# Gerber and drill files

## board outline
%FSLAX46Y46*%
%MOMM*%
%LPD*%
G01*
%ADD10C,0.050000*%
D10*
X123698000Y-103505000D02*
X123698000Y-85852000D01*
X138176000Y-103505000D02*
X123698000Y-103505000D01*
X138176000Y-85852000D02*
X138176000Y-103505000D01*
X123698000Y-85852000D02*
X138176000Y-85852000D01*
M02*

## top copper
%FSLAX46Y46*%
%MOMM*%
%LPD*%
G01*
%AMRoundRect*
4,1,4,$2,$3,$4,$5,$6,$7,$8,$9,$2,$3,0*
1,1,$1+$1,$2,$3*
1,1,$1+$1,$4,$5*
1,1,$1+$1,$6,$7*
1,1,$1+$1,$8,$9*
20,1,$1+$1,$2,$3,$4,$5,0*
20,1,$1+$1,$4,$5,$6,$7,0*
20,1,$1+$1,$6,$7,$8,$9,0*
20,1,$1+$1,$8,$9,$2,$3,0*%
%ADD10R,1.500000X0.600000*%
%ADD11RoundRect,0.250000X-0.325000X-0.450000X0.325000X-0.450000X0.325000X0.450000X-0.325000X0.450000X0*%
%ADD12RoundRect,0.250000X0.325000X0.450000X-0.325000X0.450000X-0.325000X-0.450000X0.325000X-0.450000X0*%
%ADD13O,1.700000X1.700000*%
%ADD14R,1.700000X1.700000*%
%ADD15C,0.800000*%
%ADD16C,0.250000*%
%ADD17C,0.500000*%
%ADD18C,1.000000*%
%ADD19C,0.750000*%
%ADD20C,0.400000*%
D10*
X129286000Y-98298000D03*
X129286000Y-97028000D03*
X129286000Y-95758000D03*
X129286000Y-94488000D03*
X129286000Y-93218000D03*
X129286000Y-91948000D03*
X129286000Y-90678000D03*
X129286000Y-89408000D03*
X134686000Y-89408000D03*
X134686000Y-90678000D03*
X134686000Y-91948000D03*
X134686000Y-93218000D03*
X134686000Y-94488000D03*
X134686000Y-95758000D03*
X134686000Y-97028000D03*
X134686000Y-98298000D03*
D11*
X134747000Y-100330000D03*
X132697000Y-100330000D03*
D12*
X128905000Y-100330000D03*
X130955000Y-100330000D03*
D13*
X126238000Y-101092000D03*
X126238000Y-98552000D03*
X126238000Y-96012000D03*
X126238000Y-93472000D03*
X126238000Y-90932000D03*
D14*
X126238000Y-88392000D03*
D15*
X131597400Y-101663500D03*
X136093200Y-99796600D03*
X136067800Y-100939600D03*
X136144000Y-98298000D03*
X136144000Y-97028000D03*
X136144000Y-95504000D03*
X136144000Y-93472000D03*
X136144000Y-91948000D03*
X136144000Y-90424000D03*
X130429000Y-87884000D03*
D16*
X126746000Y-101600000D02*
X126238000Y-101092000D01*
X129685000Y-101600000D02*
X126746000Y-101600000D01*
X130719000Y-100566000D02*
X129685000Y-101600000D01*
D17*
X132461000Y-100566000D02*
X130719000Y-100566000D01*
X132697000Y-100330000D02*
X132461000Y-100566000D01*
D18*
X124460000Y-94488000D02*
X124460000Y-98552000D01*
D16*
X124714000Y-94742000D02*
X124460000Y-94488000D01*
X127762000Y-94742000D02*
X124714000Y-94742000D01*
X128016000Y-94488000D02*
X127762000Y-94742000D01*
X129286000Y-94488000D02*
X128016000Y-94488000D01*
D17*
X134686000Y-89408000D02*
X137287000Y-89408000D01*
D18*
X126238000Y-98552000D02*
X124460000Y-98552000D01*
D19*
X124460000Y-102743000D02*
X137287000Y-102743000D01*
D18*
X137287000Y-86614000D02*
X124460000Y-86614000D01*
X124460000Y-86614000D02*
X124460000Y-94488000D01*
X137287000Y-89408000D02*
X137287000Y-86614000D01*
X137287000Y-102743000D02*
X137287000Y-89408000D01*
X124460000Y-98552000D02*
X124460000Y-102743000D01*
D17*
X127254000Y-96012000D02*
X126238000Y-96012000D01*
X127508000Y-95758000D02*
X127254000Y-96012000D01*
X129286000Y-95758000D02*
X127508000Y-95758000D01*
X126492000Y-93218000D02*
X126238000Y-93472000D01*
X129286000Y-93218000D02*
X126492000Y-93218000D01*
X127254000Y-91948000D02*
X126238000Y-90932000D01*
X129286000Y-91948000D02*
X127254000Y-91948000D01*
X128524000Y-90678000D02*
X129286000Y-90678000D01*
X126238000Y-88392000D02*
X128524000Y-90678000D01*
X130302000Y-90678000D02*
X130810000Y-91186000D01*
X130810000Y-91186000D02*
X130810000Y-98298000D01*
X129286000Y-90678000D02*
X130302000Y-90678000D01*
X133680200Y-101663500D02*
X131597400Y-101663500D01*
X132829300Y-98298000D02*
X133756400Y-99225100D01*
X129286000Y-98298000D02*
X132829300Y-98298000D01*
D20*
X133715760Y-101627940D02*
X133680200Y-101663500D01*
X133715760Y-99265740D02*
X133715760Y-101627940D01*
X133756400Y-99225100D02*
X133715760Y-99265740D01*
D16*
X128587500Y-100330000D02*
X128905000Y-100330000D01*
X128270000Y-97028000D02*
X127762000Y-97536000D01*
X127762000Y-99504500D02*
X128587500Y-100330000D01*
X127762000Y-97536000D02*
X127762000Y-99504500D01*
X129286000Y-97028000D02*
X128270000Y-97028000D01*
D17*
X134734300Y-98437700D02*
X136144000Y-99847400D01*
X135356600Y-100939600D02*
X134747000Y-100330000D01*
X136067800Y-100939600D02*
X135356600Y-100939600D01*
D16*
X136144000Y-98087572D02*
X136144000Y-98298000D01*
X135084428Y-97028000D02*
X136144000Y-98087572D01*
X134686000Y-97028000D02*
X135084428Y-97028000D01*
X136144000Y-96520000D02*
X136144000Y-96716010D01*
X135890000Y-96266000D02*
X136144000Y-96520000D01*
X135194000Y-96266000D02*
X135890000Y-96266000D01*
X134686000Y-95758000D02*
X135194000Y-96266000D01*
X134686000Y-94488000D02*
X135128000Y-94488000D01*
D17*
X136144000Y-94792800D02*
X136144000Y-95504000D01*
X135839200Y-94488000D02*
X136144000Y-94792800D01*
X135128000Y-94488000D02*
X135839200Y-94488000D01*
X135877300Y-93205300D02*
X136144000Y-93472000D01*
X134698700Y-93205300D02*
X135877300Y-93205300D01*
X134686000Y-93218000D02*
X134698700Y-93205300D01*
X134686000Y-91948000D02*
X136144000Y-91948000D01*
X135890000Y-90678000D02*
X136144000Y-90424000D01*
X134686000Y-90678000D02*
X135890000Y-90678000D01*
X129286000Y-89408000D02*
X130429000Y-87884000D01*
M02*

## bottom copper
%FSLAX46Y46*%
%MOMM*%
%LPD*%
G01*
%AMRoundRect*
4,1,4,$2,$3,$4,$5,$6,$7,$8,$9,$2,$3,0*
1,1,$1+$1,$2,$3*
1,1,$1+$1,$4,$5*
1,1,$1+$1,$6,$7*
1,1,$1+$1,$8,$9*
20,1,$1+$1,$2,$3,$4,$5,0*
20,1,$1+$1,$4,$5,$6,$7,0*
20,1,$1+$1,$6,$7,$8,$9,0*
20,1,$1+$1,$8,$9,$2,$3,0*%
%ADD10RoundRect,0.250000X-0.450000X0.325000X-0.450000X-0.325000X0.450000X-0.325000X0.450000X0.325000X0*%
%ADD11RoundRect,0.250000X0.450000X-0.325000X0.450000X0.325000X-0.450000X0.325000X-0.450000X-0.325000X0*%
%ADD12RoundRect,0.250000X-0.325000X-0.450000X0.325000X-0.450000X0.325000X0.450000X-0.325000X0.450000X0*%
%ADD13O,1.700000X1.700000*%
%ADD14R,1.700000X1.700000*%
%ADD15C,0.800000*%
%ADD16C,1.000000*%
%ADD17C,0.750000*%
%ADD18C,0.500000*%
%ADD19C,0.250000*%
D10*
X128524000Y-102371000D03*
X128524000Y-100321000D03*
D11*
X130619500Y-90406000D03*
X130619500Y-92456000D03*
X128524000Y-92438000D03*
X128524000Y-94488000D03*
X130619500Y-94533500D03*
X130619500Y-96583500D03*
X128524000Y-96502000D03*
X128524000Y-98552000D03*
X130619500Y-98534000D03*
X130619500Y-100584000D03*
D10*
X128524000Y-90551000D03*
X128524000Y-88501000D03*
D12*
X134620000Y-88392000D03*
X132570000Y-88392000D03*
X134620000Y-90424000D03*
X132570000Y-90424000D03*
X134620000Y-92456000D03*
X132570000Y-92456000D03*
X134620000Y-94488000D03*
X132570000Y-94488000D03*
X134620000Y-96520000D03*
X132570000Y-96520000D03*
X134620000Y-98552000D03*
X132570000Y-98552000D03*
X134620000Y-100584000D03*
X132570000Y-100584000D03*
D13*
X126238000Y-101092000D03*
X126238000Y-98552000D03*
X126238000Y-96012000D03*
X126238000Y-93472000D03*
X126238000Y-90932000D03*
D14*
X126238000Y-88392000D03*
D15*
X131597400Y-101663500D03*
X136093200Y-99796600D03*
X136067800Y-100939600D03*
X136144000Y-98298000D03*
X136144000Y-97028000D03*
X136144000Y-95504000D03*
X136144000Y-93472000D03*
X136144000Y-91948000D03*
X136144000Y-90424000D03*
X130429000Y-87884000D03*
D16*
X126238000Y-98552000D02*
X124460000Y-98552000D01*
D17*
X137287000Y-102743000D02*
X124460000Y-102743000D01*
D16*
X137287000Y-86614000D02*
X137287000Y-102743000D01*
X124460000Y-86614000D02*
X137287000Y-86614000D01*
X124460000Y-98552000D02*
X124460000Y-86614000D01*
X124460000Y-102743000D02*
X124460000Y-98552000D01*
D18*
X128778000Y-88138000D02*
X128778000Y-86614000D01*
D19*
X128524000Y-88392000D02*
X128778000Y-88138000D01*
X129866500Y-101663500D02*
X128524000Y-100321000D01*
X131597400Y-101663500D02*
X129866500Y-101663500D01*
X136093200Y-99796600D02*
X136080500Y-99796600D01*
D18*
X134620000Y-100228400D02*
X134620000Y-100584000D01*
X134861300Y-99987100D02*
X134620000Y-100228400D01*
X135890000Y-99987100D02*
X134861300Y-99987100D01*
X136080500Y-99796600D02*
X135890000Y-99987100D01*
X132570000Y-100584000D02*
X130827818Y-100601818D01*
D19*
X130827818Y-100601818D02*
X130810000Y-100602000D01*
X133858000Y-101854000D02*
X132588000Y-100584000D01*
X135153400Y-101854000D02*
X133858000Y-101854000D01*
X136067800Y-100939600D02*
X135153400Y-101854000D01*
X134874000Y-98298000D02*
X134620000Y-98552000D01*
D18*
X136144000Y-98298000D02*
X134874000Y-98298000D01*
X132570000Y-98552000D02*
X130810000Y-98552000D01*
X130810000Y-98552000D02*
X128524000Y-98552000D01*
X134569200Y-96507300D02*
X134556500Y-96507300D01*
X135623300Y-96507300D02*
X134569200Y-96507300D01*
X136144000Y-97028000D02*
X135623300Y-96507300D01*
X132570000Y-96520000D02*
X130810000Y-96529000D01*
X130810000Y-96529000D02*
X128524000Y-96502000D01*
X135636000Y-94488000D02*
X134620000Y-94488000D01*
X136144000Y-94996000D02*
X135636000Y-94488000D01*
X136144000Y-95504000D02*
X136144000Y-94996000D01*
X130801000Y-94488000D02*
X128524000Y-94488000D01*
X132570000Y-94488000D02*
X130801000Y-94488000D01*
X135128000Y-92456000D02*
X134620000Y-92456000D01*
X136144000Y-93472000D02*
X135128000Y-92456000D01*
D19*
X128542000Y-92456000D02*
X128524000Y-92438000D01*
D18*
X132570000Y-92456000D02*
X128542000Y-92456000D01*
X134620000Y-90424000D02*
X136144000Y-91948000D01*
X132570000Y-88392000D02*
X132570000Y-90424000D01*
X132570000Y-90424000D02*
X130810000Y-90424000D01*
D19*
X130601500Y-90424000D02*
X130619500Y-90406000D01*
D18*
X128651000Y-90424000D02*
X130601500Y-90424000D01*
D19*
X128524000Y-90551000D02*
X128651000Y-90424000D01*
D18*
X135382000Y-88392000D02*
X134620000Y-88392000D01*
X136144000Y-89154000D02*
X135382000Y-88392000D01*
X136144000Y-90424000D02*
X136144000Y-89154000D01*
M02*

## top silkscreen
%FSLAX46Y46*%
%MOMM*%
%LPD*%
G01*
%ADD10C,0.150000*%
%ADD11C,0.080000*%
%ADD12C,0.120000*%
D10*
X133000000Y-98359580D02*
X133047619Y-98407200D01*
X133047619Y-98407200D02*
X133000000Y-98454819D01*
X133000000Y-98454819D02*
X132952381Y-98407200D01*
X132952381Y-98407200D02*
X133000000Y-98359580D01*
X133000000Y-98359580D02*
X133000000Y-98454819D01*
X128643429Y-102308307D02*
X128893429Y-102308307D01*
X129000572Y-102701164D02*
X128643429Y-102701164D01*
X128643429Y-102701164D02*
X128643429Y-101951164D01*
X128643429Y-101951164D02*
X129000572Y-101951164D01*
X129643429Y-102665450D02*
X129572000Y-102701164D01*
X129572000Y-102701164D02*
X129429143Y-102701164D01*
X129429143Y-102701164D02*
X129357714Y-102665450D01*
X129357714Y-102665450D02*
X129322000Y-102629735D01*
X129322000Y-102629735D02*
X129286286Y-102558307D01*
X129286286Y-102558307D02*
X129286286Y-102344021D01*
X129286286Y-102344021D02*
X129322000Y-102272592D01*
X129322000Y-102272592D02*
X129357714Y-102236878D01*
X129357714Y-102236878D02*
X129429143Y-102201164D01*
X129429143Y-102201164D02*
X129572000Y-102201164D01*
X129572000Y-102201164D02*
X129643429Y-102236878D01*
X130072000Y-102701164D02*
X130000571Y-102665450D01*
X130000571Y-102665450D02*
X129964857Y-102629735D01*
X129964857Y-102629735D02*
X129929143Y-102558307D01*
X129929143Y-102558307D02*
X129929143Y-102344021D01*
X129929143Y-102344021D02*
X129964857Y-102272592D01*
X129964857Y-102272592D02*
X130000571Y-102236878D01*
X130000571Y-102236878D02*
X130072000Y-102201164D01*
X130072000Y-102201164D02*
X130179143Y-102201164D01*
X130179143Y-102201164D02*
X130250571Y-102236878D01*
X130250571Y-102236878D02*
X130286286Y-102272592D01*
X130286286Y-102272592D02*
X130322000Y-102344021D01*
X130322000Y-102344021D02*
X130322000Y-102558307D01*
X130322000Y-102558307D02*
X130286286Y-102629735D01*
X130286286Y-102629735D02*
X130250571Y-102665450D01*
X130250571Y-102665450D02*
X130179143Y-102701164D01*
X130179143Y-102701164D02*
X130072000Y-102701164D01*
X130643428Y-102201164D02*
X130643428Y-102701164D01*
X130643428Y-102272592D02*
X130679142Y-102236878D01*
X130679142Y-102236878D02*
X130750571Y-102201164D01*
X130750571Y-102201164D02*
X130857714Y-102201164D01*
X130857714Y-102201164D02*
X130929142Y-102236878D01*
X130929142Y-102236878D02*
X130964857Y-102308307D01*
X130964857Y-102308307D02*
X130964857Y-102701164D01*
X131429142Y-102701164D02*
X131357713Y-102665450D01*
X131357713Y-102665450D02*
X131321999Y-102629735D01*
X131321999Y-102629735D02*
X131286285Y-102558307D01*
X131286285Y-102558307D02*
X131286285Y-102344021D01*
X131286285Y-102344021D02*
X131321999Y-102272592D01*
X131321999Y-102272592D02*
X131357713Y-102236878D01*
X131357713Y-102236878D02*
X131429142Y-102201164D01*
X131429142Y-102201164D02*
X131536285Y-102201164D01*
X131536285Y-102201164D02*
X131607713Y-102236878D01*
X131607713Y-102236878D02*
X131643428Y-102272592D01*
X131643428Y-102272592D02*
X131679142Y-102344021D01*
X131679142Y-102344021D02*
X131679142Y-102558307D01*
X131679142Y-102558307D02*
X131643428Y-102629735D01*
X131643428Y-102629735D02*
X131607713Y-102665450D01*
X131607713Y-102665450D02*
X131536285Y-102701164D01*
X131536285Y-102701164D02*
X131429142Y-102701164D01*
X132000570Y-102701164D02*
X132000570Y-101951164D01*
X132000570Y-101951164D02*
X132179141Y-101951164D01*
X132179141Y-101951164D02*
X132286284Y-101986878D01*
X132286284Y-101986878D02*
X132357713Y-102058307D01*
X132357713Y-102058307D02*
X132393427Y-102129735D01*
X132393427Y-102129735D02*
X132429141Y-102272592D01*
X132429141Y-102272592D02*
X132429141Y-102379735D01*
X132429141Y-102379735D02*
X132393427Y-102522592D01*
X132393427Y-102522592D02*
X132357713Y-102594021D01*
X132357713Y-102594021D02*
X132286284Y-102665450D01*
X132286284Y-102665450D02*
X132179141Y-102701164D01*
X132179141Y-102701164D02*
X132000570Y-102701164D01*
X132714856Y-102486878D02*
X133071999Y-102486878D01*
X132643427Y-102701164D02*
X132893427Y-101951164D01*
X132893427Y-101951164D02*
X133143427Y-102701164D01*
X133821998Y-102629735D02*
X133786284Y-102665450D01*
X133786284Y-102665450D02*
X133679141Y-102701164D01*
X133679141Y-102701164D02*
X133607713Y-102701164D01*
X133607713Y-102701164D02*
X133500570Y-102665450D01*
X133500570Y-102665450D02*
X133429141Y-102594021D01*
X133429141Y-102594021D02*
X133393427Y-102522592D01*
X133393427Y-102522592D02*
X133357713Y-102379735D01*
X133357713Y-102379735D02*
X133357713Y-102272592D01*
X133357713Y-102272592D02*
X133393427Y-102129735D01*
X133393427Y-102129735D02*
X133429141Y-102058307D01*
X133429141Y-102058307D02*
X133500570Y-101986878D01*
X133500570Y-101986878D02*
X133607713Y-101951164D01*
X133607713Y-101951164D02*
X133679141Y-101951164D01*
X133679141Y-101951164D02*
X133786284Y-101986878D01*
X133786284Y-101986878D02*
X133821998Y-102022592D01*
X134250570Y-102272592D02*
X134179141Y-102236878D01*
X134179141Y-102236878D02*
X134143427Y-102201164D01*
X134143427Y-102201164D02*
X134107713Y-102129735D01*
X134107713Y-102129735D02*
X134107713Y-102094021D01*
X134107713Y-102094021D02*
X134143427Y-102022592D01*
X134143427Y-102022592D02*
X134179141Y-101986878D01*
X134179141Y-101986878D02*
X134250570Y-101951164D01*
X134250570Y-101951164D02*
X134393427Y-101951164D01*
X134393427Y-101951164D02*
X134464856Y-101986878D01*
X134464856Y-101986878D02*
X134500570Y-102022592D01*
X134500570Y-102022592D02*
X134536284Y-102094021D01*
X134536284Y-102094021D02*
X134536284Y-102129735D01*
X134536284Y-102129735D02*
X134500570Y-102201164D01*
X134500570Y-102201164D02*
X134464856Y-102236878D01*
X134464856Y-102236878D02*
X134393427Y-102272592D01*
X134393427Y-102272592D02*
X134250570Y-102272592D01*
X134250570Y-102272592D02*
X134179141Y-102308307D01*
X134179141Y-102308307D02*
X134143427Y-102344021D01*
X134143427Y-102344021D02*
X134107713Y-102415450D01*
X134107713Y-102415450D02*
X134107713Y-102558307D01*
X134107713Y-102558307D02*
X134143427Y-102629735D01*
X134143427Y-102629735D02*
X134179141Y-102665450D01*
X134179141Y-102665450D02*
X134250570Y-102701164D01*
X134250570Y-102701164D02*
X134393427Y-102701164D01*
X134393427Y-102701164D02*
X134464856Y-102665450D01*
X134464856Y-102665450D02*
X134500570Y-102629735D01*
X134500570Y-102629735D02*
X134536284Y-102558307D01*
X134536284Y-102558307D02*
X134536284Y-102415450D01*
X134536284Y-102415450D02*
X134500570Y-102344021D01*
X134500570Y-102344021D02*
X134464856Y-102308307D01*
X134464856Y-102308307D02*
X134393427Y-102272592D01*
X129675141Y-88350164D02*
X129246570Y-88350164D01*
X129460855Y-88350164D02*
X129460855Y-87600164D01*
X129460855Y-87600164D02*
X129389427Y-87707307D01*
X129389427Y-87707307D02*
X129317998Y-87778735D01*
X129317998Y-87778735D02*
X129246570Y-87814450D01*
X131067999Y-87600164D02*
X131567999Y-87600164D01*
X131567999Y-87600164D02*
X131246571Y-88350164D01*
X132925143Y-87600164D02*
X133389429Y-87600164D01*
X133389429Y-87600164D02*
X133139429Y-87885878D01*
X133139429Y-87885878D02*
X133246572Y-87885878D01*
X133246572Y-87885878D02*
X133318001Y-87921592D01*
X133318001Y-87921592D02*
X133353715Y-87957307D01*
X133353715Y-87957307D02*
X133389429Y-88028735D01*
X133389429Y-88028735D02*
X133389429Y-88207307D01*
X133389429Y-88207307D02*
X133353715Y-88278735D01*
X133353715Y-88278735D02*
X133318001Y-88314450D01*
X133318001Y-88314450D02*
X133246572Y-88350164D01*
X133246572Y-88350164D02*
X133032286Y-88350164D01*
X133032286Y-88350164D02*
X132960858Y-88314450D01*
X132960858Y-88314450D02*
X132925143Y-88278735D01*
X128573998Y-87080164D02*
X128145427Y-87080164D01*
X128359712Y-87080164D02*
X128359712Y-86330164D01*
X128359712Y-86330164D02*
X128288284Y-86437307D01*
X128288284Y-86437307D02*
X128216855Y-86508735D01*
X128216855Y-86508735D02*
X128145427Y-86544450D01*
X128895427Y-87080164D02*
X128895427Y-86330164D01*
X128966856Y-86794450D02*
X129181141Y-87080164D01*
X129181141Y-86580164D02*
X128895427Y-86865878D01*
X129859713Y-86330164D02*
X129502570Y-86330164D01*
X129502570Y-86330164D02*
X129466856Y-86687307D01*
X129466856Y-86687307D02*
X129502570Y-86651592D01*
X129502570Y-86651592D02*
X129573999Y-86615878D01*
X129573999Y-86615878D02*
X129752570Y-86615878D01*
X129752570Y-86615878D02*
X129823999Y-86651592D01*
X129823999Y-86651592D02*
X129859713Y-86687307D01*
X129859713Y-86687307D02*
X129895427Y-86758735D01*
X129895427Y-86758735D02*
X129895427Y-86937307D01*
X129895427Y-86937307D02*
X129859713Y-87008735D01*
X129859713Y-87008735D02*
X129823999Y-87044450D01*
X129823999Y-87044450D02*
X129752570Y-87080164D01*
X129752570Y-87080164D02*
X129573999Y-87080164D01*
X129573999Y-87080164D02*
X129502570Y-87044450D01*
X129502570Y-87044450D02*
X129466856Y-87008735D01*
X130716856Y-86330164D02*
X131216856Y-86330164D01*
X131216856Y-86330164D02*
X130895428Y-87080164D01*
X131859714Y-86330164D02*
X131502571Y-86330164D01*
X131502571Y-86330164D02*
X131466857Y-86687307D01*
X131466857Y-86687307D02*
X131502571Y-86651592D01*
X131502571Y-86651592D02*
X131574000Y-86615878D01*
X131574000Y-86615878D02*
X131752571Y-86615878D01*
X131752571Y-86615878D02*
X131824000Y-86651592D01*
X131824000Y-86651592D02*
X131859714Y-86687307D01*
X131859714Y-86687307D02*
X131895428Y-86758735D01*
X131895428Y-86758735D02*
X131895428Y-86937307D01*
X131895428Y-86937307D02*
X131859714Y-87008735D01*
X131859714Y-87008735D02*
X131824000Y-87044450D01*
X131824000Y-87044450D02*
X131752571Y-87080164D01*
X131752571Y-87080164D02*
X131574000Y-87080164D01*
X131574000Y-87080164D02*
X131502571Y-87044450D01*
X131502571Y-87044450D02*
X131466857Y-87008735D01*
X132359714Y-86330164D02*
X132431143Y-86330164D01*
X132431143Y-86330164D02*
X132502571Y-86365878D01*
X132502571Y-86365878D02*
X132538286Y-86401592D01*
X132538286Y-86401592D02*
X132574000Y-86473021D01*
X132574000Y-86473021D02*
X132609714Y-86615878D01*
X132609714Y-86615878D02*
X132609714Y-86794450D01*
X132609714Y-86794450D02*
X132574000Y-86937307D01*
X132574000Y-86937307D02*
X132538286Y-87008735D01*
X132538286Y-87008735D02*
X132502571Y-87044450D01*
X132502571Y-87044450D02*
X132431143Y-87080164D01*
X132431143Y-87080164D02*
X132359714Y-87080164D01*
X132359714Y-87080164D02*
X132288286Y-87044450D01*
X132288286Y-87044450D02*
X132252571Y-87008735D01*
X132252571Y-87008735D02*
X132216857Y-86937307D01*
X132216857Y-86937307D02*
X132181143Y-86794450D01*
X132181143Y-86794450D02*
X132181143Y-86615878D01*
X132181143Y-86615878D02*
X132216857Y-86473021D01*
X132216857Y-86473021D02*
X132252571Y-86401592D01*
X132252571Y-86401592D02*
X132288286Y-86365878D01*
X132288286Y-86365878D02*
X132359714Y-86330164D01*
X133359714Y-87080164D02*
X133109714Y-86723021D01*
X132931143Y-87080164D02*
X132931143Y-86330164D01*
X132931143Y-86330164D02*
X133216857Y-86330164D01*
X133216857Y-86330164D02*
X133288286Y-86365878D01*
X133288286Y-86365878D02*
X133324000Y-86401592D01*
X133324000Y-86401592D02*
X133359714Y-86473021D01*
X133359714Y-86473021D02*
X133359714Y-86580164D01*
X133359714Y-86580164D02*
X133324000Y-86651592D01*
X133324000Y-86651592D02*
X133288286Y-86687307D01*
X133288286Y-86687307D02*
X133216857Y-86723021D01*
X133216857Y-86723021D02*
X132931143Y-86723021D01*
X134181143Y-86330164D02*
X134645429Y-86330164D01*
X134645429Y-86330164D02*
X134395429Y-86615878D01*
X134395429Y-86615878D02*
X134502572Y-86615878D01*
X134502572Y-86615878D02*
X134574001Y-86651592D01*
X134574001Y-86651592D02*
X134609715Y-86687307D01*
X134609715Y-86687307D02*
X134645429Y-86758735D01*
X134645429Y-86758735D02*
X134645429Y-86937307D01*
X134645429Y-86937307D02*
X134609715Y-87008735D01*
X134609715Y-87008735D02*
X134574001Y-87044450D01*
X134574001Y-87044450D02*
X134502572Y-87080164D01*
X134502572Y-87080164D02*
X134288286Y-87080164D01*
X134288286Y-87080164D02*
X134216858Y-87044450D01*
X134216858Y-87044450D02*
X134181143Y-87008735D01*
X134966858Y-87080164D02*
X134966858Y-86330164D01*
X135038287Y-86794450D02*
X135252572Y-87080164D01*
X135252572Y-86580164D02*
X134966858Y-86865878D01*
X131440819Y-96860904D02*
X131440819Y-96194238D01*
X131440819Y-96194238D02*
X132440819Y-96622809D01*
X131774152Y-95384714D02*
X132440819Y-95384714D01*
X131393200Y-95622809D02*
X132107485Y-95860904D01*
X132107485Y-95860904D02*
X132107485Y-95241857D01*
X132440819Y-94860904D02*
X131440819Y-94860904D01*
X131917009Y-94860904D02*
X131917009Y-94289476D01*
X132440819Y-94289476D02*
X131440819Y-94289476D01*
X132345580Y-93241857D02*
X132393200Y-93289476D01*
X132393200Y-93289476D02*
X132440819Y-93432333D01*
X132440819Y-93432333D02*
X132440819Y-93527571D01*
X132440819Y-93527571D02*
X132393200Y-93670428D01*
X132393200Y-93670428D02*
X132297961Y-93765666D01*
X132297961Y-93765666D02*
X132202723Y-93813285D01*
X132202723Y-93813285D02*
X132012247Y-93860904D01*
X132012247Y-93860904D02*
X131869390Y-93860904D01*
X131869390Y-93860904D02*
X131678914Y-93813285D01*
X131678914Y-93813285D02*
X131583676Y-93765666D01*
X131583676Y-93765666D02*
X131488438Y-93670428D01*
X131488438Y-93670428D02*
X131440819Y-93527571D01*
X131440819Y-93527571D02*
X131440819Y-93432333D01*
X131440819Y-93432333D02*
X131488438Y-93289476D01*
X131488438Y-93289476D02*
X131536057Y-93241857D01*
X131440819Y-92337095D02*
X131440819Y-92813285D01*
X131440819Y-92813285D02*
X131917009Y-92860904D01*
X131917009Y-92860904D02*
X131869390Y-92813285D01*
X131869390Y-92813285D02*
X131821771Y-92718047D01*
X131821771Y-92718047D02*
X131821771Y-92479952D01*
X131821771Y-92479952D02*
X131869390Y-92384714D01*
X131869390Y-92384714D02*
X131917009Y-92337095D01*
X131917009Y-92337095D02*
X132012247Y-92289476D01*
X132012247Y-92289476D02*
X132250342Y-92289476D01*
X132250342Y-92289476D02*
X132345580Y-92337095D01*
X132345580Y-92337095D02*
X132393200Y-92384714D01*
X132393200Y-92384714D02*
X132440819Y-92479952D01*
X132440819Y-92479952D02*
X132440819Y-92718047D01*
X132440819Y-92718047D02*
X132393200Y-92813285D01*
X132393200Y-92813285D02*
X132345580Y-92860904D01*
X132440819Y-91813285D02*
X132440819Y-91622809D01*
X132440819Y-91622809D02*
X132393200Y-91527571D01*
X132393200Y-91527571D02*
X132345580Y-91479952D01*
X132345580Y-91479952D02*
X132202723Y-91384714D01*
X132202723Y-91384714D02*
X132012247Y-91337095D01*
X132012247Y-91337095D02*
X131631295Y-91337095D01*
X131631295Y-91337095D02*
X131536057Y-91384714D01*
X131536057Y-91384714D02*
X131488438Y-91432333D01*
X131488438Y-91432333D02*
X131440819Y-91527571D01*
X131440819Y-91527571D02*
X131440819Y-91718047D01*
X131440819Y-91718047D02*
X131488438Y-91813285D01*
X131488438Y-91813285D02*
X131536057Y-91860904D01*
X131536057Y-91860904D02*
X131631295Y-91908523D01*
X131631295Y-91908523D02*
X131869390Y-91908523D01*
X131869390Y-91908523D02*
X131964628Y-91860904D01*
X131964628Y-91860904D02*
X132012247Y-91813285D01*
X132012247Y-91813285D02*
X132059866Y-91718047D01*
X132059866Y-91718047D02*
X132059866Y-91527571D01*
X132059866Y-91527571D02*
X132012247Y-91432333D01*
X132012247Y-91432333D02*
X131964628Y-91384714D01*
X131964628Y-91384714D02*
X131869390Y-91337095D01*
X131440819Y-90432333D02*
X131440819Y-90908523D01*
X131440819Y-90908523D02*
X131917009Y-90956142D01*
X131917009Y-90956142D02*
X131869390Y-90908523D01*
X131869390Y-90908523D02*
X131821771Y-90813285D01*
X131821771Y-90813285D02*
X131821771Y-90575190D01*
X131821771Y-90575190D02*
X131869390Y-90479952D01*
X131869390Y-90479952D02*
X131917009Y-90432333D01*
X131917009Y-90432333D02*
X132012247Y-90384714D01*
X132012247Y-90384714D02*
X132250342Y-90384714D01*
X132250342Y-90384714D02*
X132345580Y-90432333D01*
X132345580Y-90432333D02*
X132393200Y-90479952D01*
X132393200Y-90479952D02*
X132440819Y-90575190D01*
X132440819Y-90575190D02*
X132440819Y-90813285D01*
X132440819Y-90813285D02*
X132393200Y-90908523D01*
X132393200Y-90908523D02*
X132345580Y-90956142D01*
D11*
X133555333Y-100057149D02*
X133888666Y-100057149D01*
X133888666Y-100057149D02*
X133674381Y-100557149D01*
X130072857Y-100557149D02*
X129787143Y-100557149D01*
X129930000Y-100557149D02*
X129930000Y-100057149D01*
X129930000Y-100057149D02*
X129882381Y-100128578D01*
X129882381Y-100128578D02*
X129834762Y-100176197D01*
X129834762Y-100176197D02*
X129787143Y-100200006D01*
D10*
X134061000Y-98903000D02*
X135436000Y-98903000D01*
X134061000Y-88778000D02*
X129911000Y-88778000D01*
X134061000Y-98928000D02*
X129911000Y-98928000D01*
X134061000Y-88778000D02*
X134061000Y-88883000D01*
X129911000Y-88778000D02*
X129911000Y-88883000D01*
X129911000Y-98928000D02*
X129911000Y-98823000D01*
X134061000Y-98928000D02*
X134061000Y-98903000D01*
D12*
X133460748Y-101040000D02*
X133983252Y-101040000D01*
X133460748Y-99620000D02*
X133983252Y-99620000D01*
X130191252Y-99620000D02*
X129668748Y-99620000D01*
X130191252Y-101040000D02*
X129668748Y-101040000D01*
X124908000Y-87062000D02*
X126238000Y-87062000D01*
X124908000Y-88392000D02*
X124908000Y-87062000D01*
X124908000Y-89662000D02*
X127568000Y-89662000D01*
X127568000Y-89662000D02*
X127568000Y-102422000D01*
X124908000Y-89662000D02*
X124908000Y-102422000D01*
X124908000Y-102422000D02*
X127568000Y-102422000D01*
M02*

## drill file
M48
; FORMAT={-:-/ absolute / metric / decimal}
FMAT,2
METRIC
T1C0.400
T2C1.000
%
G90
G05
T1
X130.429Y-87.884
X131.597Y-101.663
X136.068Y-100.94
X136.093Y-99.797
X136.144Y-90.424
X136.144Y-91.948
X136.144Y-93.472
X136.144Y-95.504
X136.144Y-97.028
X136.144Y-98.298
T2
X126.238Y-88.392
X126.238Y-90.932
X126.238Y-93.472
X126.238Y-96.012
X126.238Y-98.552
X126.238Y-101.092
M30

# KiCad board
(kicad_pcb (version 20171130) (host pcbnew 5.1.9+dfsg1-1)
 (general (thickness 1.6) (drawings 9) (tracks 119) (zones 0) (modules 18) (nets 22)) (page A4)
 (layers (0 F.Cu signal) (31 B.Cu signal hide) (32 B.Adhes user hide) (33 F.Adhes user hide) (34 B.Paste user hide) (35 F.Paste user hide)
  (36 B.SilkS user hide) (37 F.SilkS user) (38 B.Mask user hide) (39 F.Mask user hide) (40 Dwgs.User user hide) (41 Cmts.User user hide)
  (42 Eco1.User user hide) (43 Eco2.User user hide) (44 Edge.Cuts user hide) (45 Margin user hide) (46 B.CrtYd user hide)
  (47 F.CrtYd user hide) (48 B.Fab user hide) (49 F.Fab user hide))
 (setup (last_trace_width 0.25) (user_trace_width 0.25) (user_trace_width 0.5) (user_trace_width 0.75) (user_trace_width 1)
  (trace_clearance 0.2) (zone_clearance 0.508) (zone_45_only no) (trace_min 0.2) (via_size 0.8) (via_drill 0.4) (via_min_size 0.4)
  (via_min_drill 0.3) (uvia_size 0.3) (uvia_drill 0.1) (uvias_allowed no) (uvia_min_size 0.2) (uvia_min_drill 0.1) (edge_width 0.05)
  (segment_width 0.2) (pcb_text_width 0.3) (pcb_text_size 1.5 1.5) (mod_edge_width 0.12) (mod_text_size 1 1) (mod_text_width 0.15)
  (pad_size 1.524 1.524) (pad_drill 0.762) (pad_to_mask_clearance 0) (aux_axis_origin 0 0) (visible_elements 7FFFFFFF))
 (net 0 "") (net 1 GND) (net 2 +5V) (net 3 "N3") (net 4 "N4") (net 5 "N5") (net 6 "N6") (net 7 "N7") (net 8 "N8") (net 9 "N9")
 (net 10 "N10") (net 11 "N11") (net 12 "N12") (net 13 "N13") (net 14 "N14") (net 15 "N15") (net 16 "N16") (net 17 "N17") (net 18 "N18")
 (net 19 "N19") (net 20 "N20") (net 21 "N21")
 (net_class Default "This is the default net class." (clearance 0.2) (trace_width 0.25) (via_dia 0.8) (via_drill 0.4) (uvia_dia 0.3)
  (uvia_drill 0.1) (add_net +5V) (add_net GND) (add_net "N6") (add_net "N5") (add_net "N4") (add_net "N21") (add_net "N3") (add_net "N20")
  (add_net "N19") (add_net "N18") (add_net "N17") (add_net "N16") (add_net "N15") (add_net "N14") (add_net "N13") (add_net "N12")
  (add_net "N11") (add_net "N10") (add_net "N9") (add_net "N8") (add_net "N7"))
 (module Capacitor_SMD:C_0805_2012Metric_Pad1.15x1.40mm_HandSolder (layer B.Cu) (at 128.524 101.346 270)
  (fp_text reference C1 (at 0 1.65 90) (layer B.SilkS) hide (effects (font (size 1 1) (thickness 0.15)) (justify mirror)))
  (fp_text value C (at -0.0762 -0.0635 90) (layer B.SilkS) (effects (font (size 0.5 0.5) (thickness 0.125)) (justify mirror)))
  (pad 2 smd roundrect (at 1.025 0 270) (size 1.15 1.4) (layers B.Cu B.Paste B.Mask) (roundrect_rratio 0.217391) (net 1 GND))
  (pad 1 smd roundrect (at -1.025 0 270) (size 1.15 1.4) (layers B.Cu B.Paste B.Mask) (roundrect_rratio 0.217391) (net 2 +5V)))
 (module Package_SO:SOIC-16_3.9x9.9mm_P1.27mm (layer F.Cu) (at 131.986 93.853 180)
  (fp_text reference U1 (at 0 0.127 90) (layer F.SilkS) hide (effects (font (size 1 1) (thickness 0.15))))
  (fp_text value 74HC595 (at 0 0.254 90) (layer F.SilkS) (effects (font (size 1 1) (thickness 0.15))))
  (fp_line (start -2.075 -5.05) (end -3.45 -5.05) (layer F.SilkS) (width 0.15))
  (fp_line (start -2.075 5.075) (end 2.075 5.075) (layer F.SilkS) (width 0.15))
  (fp_line (start -2.075 -5.075) (end 2.075 -5.075) (layer F.SilkS) (width 0.15))
  (fp_line (start -2.075 5.075) (end -2.075 4.97) (layer F.SilkS) (width 0.15))
  (fp_line (start 2.075 5.075) (end 2.075 4.97) (layer F.SilkS) (width 0.15))
  (fp_line (start 2.075 -5.075) (end 2.075 -4.97) (layer F.SilkS) (width 0.15))
  (fp_line (start -2.075 -5.075) (end -2.075 -5.05) (layer F.SilkS) (width 0.15))
  (pad 16 smd rect (at 2.7 -4.445 180) (size 1.5 0.6) (layers F.Cu F.Paste F.Mask) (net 2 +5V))
  (pad 15 smd rect (at 2.7 -3.175 180) (size 1.5 0.6) (layers F.Cu F.Paste F.Mask) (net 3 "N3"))
  (pad 14 smd rect (at 2.7 -1.905 180) (size 1.5 0.6) (layers F.Cu F.Paste F.Mask) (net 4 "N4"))
  (pad 13 smd rect (at 2.7 -0.635 180) (size 1.5 0.6) (layers F.Cu F.Paste F.Mask) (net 1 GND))
  (pad 12 smd rect (at 2.7 0.635 180) (size 1.5 0.6) (layers F.Cu F.Paste F.Mask) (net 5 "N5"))
  (pad 11 smd rect (at 2.7 1.905 180) (size 1.5 0.6) (layers F.Cu F.Paste F.Mask) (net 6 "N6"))
  (pad 10 smd rect (at 2.7 3.175 180) (size 1.5 0.6) (layers F.Cu F.Paste F.Mask) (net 2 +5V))
  (pad 9 smd rect (at 2.7 4.445 180) (size 1.5 0.6) (layers F.Cu F.Paste F.Mask) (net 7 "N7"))
  (pad 8 smd rect (at -2.7 4.445 180) (size 1.5 0.6) (layers F.Cu F.Paste F.Mask) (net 1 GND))
  (pad 7 smd rect (at -2.7 3.175 180) (size 1.5 0.6) (layers F.Cu F.Paste F.Mask) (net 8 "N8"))
  (pad 6 smd rect (at -2.7 1.905 180) (size 1.5 0.6) (layers F.Cu F.Paste F.Mask) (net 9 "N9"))
  (pad 5 smd rect (at -2.7 0.635 180) (size 1.5 0.6) (layers F.Cu F.Paste F.Mask) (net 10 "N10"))
  (pad 4 smd rect (at -2.7 -0.635 180) (size 1.5 0.6) (layers F.Cu F.Paste F.Mask) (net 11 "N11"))
  (pad 3 smd rect (at -2.7 -1.905 180) (size 1.5 0.6) (layers F.Cu F.Paste F.Mask) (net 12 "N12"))
  (pad 2 smd rect (at -2.7 -3.175 180) (size 1.5 0.6) (layers F.Cu F.Paste F.Mask) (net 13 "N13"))
  (pad 1 smd rect (at -2.7 -4.445 180) (size 1.5 0.6) (layers F.Cu F.Paste F.Mask) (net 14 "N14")))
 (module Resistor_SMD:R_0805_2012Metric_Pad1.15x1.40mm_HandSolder (layer B.Cu) (at 130.6195 91.431 90)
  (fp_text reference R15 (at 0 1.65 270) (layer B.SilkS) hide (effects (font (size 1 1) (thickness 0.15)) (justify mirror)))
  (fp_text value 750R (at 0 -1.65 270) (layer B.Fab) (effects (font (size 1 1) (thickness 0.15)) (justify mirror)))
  (pad 2 smd roundrect (at 1.025 0 90) (size 1.15 1.4) (layers B.Cu B.Paste B.Mask) (roundrect_rratio 0.217391) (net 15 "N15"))
  (pad 1 smd roundrect (at -1.025 0 90) (size 1.15 1.4) (layers B.Cu B.Paste B.Mask) (roundrect_rratio 0.217391) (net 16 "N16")))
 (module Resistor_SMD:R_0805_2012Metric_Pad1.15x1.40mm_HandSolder (layer B.Cu) (at 128.524 93.463 90)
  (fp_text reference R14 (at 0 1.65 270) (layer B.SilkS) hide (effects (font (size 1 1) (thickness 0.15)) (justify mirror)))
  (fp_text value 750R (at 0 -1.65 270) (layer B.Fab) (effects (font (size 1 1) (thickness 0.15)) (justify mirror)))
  (pad 2 smd roundrect (at 1.025 0 90) (size 1.15 1.4) (layers B.Cu B.Paste B.Mask) (roundrect_rratio 0.217391) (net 16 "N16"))
  (pad 1 smd roundrect (at -1.025 0 90) (size 1.15 1.4) (layers B.Cu B.Paste B.Mask) (roundrect_rratio 0.217391) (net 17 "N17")))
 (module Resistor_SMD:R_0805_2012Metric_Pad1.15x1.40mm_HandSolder (layer B.Cu) (at 130.6195 95.5585 90)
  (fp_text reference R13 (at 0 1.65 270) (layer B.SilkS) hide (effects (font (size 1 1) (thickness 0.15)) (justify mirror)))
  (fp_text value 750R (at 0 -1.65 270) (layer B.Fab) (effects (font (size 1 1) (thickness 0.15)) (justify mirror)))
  (pad 2 smd roundrect (at 1.025 0 90) (size 1.15 1.4) (layers B.Cu B.Paste B.Mask) (roundrect_rratio 0.217391) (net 17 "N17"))
  (pad 1 smd roundrect (at -1.025 0 90) (size 1.15 1.4) (layers B.Cu B.Paste B.Mask) (roundrect_rratio 0.217391) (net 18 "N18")))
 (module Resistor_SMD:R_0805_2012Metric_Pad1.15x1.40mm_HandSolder (layer B.Cu) (at 128.524 97.527 90)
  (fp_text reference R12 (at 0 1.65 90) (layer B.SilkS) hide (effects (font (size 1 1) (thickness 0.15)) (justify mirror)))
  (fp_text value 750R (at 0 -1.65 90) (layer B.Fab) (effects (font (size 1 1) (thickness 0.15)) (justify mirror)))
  (pad 2 smd roundrect (at 1.025 0 90) (size 1.15 1.4) (layers B.Cu B.Paste B.Mask) (roundrect_rratio 0.217391) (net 18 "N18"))
  (pad 1 smd roundrect (at -1.025 0 90) (size 1.15 1.4) (layers B.Cu B.Paste B.Mask) (roundrect_rratio 0.217391) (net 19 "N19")))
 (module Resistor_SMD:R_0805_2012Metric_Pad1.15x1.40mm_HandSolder (layer B.Cu) (at 130.6195 99.559 90)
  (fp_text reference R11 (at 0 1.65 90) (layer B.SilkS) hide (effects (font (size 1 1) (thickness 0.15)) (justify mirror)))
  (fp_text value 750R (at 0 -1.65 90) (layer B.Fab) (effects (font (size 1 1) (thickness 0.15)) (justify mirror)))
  (pad 2 smd roundrect (at 1.025 0 90) (size 1.15 1.4) (layers B.Cu B.Paste B.Mask) (roundrect_rratio 0.217391) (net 19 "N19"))
  (pad 1 smd roundrect (at -1.025 0 90) (size 1.15 1.4) (layers B.Cu B.Paste B.Mask) (roundrect_rratio 0.217391) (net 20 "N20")))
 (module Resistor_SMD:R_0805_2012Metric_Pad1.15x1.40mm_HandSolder (layer F.Cu) (at 133.722 100.33)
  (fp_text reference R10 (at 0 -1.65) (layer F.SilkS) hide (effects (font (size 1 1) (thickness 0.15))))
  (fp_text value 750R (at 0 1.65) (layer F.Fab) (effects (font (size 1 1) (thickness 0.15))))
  (fp_line (start -0.261252 0.71) (end 0.261252 0.71) (layer F.SilkS) (width 0.12))
  (fp_line (start -0.261252 -0.71) (end 0.261252 -0.71) (layer F.SilkS) (width 0.12))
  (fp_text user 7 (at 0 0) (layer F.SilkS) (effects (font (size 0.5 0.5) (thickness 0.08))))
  (pad 2 smd roundrect (at 1.025 0) (size 1.15 1.4) (layers F.Cu F.Paste F.Mask) (roundrect_rratio 0.217391) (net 20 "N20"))
  (pad 1 smd roundrect (at -1.025 0) (size 1.15 1.4) (layers F.Cu F.Paste F.Mask) (roundrect_rratio 0.217391) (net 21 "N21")))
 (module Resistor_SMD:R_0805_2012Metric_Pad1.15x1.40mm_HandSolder (layer B.Cu) (at 128.524 89.526 270)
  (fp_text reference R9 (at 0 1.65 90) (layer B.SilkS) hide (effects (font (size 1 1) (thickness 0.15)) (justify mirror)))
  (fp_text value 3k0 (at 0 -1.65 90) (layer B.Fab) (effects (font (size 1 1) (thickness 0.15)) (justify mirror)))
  (pad 2 smd roundrect (at 1.025 0 270) (size 1.15 1.4) (layers B.Cu B.Paste B.Mask) (roundrect_rratio 0.217391) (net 15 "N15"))
  (pad 1 smd roundrect (at -1.025 0 270) (size 1.15 1.4) (layers B.Cu B.Paste B.Mask) (roundrect_rratio 0.217391) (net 1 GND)))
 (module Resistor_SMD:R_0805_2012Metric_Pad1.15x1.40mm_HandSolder (layer B.Cu) (at 133.595 88.392)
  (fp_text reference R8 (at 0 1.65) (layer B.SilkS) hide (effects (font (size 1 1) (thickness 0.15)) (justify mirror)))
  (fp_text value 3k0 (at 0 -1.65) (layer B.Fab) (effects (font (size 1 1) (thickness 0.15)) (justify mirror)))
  (pad 2 smd roundrect (at 1.025 0) (size 1.15 1.4) (layers B.Cu B.Paste B.Mask) (roundrect_rratio 0.217391) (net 8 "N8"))
  (pad 1 smd roundrect (at -1.025 0) (size 1.15 1.4) (layers B.Cu B.Paste B.Mask) (roundrect_rratio 0.217391) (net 15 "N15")))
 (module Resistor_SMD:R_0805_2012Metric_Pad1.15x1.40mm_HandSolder (layer B.Cu) (at 133.595 90.424)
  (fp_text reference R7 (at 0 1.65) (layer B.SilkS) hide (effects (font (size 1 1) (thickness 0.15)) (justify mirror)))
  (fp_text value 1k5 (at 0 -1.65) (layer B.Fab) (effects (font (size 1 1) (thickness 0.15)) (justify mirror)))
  (pad 2 smd roundrect (at 1.025 0) (size 1.15 1.4) (layers B.Cu B.Paste B.Mask) (roundrect_rratio 0.217391) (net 9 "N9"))
  (pad 1 smd roundrect (at -1.025 0) (size 1.15 1.4) (layers B.Cu B.Paste B.Mask) (roundrect_rratio 0.217391) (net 15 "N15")))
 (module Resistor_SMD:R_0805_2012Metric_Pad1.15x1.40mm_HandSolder (layer B.Cu) (at 133.595 92.456)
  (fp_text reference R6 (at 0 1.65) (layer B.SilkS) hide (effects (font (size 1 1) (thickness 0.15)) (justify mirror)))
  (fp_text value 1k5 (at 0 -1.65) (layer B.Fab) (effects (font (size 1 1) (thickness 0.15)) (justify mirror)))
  (pad 2 smd roundrect (at 1.025 0) (size 1.15 1.4) (layers B.Cu B.Paste B.Mask) (roundrect_rratio 0.217391) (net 10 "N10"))
  (pad 1 smd roundrect (at -1.025 0) (size 1.15 1.4) (layers B.Cu B.Paste B.Mask) (roundrect_rratio 0.217391) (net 16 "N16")))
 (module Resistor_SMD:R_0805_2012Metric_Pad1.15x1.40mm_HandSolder (layer B.Cu) (at 133.595 94.488)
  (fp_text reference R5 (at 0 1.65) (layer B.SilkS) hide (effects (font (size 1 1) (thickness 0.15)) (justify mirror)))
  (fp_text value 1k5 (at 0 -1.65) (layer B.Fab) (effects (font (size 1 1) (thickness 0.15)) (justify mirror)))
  (pad 2 smd roundrect (at 1.025 0) (size 1.15 1.4) (layers B.Cu B.Paste B.Mask) (roundrect_rratio 0.217391) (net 11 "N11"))
  (pad 1 smd roundrect (at -1.025 0) (size 1.15 1.4) (layers B.Cu B.Paste B.Mask) (roundrect_rratio 0.217391) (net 17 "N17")))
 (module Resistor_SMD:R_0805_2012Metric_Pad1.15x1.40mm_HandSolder (layer B.Cu) (at 133.595 96.52)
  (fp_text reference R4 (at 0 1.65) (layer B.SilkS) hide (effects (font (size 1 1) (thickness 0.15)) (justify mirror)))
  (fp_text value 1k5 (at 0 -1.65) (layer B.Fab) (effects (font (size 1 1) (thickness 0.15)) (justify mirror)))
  (pad 2 smd roundrect (at 1.025 0) (size 1.15 1.4) (layers B.Cu B.Paste B.Mask) (roundrect_rratio 0.217391) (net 12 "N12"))
  (pad 1 smd roundrect (at -1.025 0) (size 1.15 1.4) (layers B.Cu B.Paste B.Mask) (roundrect_rratio 0.217391) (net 18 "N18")))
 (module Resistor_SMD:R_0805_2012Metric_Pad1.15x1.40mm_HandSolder (layer B.Cu) (at 133.595 98.552)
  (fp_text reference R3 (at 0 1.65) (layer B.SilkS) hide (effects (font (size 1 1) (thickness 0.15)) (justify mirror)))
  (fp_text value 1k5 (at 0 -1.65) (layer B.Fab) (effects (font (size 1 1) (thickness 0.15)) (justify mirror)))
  (pad 2 smd roundrect (at 1.025 0) (size 1.15 1.4) (layers B.Cu B.Paste B.Mask) (roundrect_rratio 0.217391) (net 13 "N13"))
  (pad 1 smd roundrect (at -1.025 0) (size 1.15 1.4) (layers B.Cu B.Paste B.Mask) (roundrect_rratio 0.217391) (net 19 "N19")))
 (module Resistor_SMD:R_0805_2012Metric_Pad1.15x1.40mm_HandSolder (layer B.Cu) (at 133.595 100.584)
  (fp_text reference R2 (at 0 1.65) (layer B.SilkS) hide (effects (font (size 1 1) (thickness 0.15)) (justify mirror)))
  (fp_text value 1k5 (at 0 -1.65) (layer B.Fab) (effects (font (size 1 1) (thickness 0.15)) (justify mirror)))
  (pad 2 smd roundrect (at 1.025 0) (size 1.15 1.4) (layers B.Cu B.Paste B.Mask) (roundrect_rratio 0.217391) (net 14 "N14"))
  (pad 1 smd roundrect (at -1.025 0) (size 1.15 1.4) (layers B.Cu B.Paste B.Mask) (roundrect_rratio 0.217391) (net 20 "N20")))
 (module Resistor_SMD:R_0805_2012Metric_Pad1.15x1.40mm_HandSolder (layer F.Cu) (at 129.93 100.33 180)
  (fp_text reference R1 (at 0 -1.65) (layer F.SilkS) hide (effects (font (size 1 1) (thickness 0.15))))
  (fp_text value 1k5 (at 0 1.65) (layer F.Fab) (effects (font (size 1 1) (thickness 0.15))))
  (fp_line (start -0.261252 0.71) (end 0.261252 0.71) (layer F.SilkS) (width 0.12))
  (fp_line (start -0.261252 -0.71) (end 0.261252 -0.71) (layer F.SilkS) (width 0.12))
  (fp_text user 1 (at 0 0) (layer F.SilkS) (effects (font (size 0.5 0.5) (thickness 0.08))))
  (pad 2 smd roundrect (at 1.025 0 180) (size 1.15 1.4) (layers F.Cu F.Paste F.Mask) (roundrect_rratio 0.217391) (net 3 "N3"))
  (pad 1 smd roundrect (at -1.025 0 180) (size 1.15 1.4) (layers F.Cu F.Paste F.Mask) (roundrect_rratio 0.217391) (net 21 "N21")))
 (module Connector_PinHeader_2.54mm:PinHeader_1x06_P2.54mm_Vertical (layer F.Cu) (at 126.238 88.392)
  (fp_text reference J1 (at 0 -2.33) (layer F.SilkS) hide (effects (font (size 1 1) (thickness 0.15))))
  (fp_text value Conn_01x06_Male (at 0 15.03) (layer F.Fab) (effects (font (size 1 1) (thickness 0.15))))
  (fp_line (start -1.33 -1.33) (end 0 -1.33) (layer F.SilkS) (width 0.12))
  (fp_line (start -1.33 0) (end -1.33 -1.33) (layer F.SilkS) (width 0.12))
  (fp_line (start -1.33 1.27) (end 1.33 1.27) (layer F.SilkS) (width 0.12))
  (fp_line (start 1.33 1.27) (end 1.33 14.03) (layer F.SilkS) (width 0.12))
  (fp_line (start -1.33 1.27) (end -1.33 14.03) (layer F.SilkS) (width 0.12))
  (fp_line (start -1.33 14.03) (end 1.33 14.03) (layer F.SilkS) (width 0.12))
  (pad 6 thru_hole oval (at 0 12.7) (size 1.7 1.7) (drill 1) (layers *.Cu *.Mask) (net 21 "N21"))
  (pad 5 thru_hole oval (at 0 10.16) (size 1.7 1.7) (drill 1) (layers *.Cu *.Mask) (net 1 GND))
  (pad 4 thru_hole oval (at 0 7.62) (size 1.7 1.7) (drill 1) (layers *.Cu *.Mask) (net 4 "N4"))
  (pad 3 thru_hole oval (at 0 5.08) (size 1.7 1.7) (drill 1) (layers *.Cu *.Mask) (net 5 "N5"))
  (pad 2 thru_hole oval (at 0 2.54) (size 1.7 1.7) (drill 1) (layers *.Cu *.Mask) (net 6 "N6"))
  (pad 1 thru_hole rect (at 0 0) (size 1.7 1.7) (drill 1) (layers *.Cu *.Mask) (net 2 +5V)))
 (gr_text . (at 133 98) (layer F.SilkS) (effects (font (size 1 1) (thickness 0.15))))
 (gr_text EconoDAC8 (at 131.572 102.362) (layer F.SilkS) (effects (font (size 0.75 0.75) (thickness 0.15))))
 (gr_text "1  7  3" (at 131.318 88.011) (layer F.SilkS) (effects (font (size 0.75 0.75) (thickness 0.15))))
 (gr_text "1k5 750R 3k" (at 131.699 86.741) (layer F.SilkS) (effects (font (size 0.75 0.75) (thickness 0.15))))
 (gr_line (start 123.698 103.505) (end 123.698 85.852) (layer Edge.Cuts) (width 0.05))
 (gr_line (start 138.176 103.505) (end 123.698 103.505) (layer Edge.Cuts) (width 0.05))
 (gr_line (start 138.176 85.852) (end 138.176 103.505) (layer Edge.Cuts) (width 0.05))
 (gr_line (start 123.698 85.852) (end 138.176 85.852) (layer Edge.Cuts) (width 0.05))
 (segment (start 126.746 101.6) (end 126.238 101.092) (width 0.25) (layer F.Cu) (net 21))
 (segment (start 129.685 101.6) (end 126.746 101.6) (width 0.25) (layer F.Cu) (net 21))
 (segment (start 130.719 100.566) (end 129.685 101.6) (width 0.25) (layer F.Cu) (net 21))
 (segment (start 132.461 100.566) (end 130.719 100.566) (width 0.5) (layer F.Cu) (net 21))
 (segment (start 132.697 100.33) (end 132.461 100.566) (width 0.5) (layer F.Cu) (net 21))
 (segment (start 124.46 94.488) (end 124.46 98.552) (width 1) (layer F.Cu) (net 1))
 (segment (start 124.714 94.742) (end 124.46 94.488) (width 0.25) (layer F.Cu) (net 1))
 (segment (start 127.762 94.742) (end 124.714 94.742) (width 0.25) (layer F.Cu) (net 1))
 (segment (start 128.016 94.488) (end 127.762 94.742) (width 0.25) (layer F.Cu) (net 1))
 (segment (start 129.286 94.488) (end 128.016 94.488) (width 0.25) (layer F.Cu) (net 1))
 (segment (start 134.686 89.408) (end 137.287 89.408) (width 0.5) (layer F.Cu) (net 1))
 (segment (start 126.238 98.552) (end 124.46 98.552) (width 1) (layer F.Cu) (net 1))
 (segment (start 126.238 98.552) (end 124.46 98.552) (width 1) (layer B.Cu) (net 1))
 (segment (start 124.46 102.743) (end 137.287 102.743) (width 0.75) (layer F.Cu) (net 1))
 (segment (start 137.287 86.614) (end 124.46 86.614) (width 1) (layer F.Cu) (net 1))
 (segment (start 124.46 86.614) (end 124.46 94.488) (width 1) (layer F.Cu) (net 1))
 (segment (start 137.287 89.408) (end 137.287 86.614) (width 1) (layer F.Cu) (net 1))
 (segment (start 137.287 102.743) (end 124.46 102.743) (width 0.75) (layer B.Cu) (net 1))
 (segment (start 137.287 102.743) (end 137.287 89.408) (width 1) (layer F.Cu) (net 1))
 (segment (start 137.287 86.614) (end 137.287 102.743) (width 1) (layer B.Cu) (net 1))
 (segment (start 124.46 86.614) (end 137.287 86.614) (width 1) (layer B.Cu) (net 1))
 (segment (start 124.46 98.552) (end 124.46 86.614) (width 1) (layer B.Cu) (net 1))
 (segment (start 124.46 98.552) (end 124.46 102.743) (width 1) (layer F.Cu) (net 1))
 (segment (start 124.46 102.743) (end 124.46 98.552) (width 1) (layer B.Cu) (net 1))
 (segment (start 128.778 88.138) (end 128.778 86.614) (width 0.5) (layer B.Cu) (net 1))
 (segment (start 128.524 88.392) (end 128.778 88.138) (width 0.25) (layer B.Cu) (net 1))
 (segment (start 127.254 96.012) (end 126.238 96.012) (width 0.5) (layer F.Cu) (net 4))
 (segment (start 127.508 95.758) (end 127.254 96.012) (width 0.5) (layer F.Cu) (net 4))
 (segment (start 129.286 95.758) (end 127.508 95.758) (width 0.5) (layer F.Cu) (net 4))
 (segment (start 126.492 93.218) (end 126.238 93.472) (width 0.5) (layer F.Cu) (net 5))
 (segment (start 129.286 93.218) (end 126.492 93.218) (width 0.5) (layer F.Cu) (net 5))
 (segment (start 127.254 91.948) (end 126.238 90.932) (width 0.5) (layer F.Cu) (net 6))
 (segment (start 129.286 91.948) (end 127.254 91.948) (width 0.5) (layer F.Cu) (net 6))
 (via (at 131.5974 101.6635) (size 0.8) (drill 0.4) (layers F.Cu B.Cu) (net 2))
 (segment (start 128.524 90.678) (end 129.286 90.678) (width 0.5) (layer F.Cu) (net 2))
 (segment (start 126.238 88.392) (end 128.524 90.678) (width 0.5) (layer F.Cu) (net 2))
 (segment (start 129.8665 101.6635) (end 128.524 100.321) (width 0.25) (layer B.Cu) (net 2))
 (segment (start 131.5974 101.6635) (end 129.8665 101.6635) (width 0.25) (layer B.Cu) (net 2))
 (segment (start 130.302 90.678) (end 130.81 91.186) (width 0.5) (layer F.Cu) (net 2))
 (segment (start 130.81 91.186) (end 130.81 98.298) (width 0.5) (layer F.Cu) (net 2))
 (segment (start 129.286 90.678) (end 130.302 90.678) (width 0.5) (layer F.Cu) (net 2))
 (segment (start 133.6802 101.6635) (end 131.5974 101.6635) (width 0.5) (layer F.Cu) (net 2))
 (segment (start 132.8293 98.298) (end 133.7564 99.2251) (width 0.5) (layer F.Cu) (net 2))
 (segment (start 129.286 98.298) (end 132.8293 98.298) (width 0.5) (layer F.Cu) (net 2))
 (segment (start 133.71576 101.62794) (end 133.6802 101.6635) (width 0.4) (layer F.Cu) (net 2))
 (segment (start 133.71576 99.26574) (end 133.71576 101.62794) (width 0.4) (layer F.Cu) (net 2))
 (segment (start 133.7564 99.2251) (end 133.71576 99.26574) (width 0.4) (layer F.Cu) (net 2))
 (segment (start 128.5875 100.33) (end 128.905 100.33) (width 0.25) (layer F.Cu) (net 3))
 (segment (start 128.27 97.028) (end 127.762 97.536) (width 0.25) (layer F.Cu) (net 3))
 (segment (start 127.762 99.5045) (end 128.5875 100.33) (width 0.25) (layer F.Cu) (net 3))
 (segment (start 127.762 97.536) (end 127.762 99.5045) (width 0.25) (layer F.Cu) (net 3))
 (segment (start 129.286 97.028) (end 128.27 97.028) (width 0.25) (layer F.Cu) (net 3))
 (via (at 136.0932 99.7966) (size 0.8) (drill 0.4) (layers F.Cu B.Cu) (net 14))
 (segment (start 136.0932 99.7966) (end 136.0805 99.7966) (width 0.25) (layer B.Cu) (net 14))
 (segment (start 134.62 100.2284) (end 134.62 100.584) (width 0.5) (layer B.Cu) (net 14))
 (segment (start 134.8613 99.9871) (end 134.62 100.2284) (width 0.5) (layer B.Cu) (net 14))
 (segment (start 135.89 99.9871) (end 134.8613 99.9871) (width 0.5) (layer B.Cu) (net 14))
 (segment (start 136.0805 99.7966) (end 135.89 99.9871) (width 0.5) (layer B.Cu) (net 14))
 (segment (start 134.7343 98.4377) (end 136.144 99.8474) (width 0.5) (layer F.Cu) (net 14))
 (segment (start 132.57 100.584) (end 130.827818 100.601818) (width 0.5) (layer B.Cu) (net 20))
 (segment (start 130.827818 100.601818) (end 130.81 100.602) (width 0.25) (layer B.Cu) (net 20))
 (via (at 136.0678 100.9396) (size 0.8) (drill 0.4) (layers F.Cu B.Cu) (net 20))
 (segment (start 135.3566 100.9396) (end 134.747 100.33) (width 0.5) (layer F.Cu) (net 20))
 (segment (start 136.0678 100.9396) (end 135.3566 100.9396) (width 0.5) (layer F.Cu) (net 20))
 (segment (start 133.858 101.854) (end 132.588 100.584) (width 0.25) (layer B.Cu) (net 20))
 (segment (start 135.1534 101.854) (end 133.858 101.854) (width 0.25) (layer B.Cu) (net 20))
 (segment (start 136.0678 100.9396) (end 135.1534 101.854) (width 0.25) (layer B.Cu) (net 20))
 (via (at 136.144 98.298) (size 0.8) (drill 0.4) (layers F.Cu B.Cu) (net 13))
 (segment (start 134.874 98.298) (end 134.62 98.552) (width 0.25) (layer B.Cu) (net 13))
 (segment (start 136.144 98.298) (end 134.874 98.298) (width 0.5) (layer B.Cu) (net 13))
 (segment (start 136.144 98.087572) (end 136.144 98.298) (width 0.25) (layer F.Cu) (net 13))
 (segment (start 135.084428 97.028) (end 136.144 98.087572) (width 0.25) (layer F.Cu) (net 13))
 (segment (start 134.686 97.028) (end 135.084428 97.028) (width 0.25) (layer F.Cu) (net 13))
 (segment (start 132.57 98.552) (end 130.81 98.552) (width 0.5) (layer B.Cu) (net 19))
 (segment (start 130.81 98.552) (end 128.524 98.552) (width 0.5) (layer B.Cu) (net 19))
 (via (at 136.144 97.028) (size 0.8) (drill 0.4) (layers F.Cu B.Cu) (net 12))
 (segment (start 136.144 96.52) (end 136.144 96.71601) (width 0.25) (layer F.Cu) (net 12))
 (segment (start 135.89 96.266) (end 136.144 96.52) (width 0.25) (layer F.Cu) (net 12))
 (segment (start 135.194 96.266) (end 135.89 96.266) (width 0.25) (layer F.Cu) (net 12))
 (segment (start 134.686 95.758) (end 135.194 96.266) (width 0.25) (layer F.Cu) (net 12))
 (segment (start 134.5692 96.5073) (end 134.5565 96.5073) (width 0.5) (layer B.Cu) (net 12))
 (segment (start 135.6233 96.5073) (end 134.5692 96.5073) (width 0.5) (layer B.Cu) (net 12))
 (segment (start 136.144 97.028) (end 135.6233 96.5073) (width 0.5) (layer B.Cu) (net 12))
 (segment (start 132.57 96.52) (end 130.81 96.529) (width 0.5) (layer B.Cu) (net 18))
 (segment (start 130.81 96.529) (end 128.524 96.502) (width 0.5) (layer B.Cu) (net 18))
 (via (at 136.144 95.504) (size 0.8) (drill 0.4) (layers F.Cu B.Cu) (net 11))
 (segment (start 134.686 94.488) (end 135.128 94.488) (width 0.25) (layer F.Cu) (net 11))
 (segment (start 135.636 94.488) (end 134.62 94.488) (width 0.5) (layer B.Cu) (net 11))
 (segment (start 136.144 94.996) (end 135.636 94.488) (width 0.5) (layer B.Cu) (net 11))
 (segment (start 136.144 95.504) (end 136.144 94.996) (width 0.5) (layer B.Cu) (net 11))
 (segment (start 136.144 94.7928) (end 136.144 95.504) (width 0.5) (layer F.Cu) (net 11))
 (segment (start 135.8392 94.488) (end 136.144 94.7928) (width 0.5) (layer F.Cu) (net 11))
 (segment (start 135.128 94.488) (end 135.8392 94.488) (width 0.5) (layer F.Cu) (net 11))
 (segment (start 130.801 94.488) (end 128.524 94.488) (width 0.5) (layer B.Cu) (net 17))
 (segment (start 132.57 94.488) (end 130.801 94.488) (width 0.5) (layer B.Cu) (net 17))
 (via (at 136.144 93.472) (size 0.8) (drill 0.4) (layers F.Cu B.Cu) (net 10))
 (segment (start 135.128 92.456) (end 134.62 92.456) (width 0.5) (layer B.Cu) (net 10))
 (segment (start 136.144 93.472) (end 135.128 92.456) (width 0.5) (layer B.Cu) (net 10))
 (segment (start 135.8773 93.2053) (end 136.144 93.472) (width 0.5) (layer F.Cu) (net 10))
 (segment (start 134.6987 93.2053) (end 135.8773 93.2053) (width 0.5) (layer F.Cu) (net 10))
 (segment (start 134.686 93.218) (end 134.6987 93.2053) (width 0.5) (layer F.Cu) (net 10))
 (segment (start 128.542 92.456) (end 128.524 92.438) (width 0.25) (layer B.Cu) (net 16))
 (segment (start 132.57 92.456) (end 128.542 92.456) (width 0.5) (layer B.Cu) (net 16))
 (via (at 136.144 91.948) (size 0.8) (drill 0.4) (layers F.Cu B.Cu) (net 9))
 (segment (start 134.62 90.424) (end 136.144 91.948) (width 0.5) (layer B.Cu) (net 9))
 (segment (start 134.686 91.948) (end 136.144 91.948) (width 0.5) (layer F.Cu) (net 9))
 (segment (start 132.57 88.392) (end 132.57 90.424) (width 0.5) (layer B.Cu) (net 15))
 (segment (start 132.57 90.424) (end 130.81 90.424) (width 0.5) (layer B.Cu) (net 15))
 (segment (start 130.6015 90.424) (end 130.6195 90.406) (width 0.25) (layer B.Cu) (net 15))
 (segment (start 128.651 90.424) (end 130.6015 90.424) (width 0.5) (layer B.Cu) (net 15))
 (segment (start 128.524 90.551) (end 128.651 90.424) (width 0.25) (layer B.Cu) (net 15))
 (via (at 136.144 90.424) (size 0.8) (drill 0.4) (layers F.Cu B.Cu) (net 8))
 (segment (start 135.382 88.392) (end 134.62 88.392) (width 0.5) (layer B.Cu) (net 8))
 (segment (start 136.144 89.154) (end 135.382 88.392) (width 0.5) (layer B.Cu) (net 8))
 (segment (start 136.144 90.424) (end 136.144 89.154) (width 0.5) (layer B.Cu) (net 8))
 (segment (start 135.89 90.678) (end 136.144 90.424) (width 0.5) (layer F.Cu) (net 8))
 (segment (start 134.686 90.678) (end 135.89 90.678) (width 0.5) (layer F.Cu) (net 8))
 (via (at 130.429 87.884) (size 0.8) (drill 0.4) (layers F.Cu B.Cu) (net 7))
 (segment (start 129.286 89.408) (end 130.429 87.884) (width 0.5) (layer F.Cu) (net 7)))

